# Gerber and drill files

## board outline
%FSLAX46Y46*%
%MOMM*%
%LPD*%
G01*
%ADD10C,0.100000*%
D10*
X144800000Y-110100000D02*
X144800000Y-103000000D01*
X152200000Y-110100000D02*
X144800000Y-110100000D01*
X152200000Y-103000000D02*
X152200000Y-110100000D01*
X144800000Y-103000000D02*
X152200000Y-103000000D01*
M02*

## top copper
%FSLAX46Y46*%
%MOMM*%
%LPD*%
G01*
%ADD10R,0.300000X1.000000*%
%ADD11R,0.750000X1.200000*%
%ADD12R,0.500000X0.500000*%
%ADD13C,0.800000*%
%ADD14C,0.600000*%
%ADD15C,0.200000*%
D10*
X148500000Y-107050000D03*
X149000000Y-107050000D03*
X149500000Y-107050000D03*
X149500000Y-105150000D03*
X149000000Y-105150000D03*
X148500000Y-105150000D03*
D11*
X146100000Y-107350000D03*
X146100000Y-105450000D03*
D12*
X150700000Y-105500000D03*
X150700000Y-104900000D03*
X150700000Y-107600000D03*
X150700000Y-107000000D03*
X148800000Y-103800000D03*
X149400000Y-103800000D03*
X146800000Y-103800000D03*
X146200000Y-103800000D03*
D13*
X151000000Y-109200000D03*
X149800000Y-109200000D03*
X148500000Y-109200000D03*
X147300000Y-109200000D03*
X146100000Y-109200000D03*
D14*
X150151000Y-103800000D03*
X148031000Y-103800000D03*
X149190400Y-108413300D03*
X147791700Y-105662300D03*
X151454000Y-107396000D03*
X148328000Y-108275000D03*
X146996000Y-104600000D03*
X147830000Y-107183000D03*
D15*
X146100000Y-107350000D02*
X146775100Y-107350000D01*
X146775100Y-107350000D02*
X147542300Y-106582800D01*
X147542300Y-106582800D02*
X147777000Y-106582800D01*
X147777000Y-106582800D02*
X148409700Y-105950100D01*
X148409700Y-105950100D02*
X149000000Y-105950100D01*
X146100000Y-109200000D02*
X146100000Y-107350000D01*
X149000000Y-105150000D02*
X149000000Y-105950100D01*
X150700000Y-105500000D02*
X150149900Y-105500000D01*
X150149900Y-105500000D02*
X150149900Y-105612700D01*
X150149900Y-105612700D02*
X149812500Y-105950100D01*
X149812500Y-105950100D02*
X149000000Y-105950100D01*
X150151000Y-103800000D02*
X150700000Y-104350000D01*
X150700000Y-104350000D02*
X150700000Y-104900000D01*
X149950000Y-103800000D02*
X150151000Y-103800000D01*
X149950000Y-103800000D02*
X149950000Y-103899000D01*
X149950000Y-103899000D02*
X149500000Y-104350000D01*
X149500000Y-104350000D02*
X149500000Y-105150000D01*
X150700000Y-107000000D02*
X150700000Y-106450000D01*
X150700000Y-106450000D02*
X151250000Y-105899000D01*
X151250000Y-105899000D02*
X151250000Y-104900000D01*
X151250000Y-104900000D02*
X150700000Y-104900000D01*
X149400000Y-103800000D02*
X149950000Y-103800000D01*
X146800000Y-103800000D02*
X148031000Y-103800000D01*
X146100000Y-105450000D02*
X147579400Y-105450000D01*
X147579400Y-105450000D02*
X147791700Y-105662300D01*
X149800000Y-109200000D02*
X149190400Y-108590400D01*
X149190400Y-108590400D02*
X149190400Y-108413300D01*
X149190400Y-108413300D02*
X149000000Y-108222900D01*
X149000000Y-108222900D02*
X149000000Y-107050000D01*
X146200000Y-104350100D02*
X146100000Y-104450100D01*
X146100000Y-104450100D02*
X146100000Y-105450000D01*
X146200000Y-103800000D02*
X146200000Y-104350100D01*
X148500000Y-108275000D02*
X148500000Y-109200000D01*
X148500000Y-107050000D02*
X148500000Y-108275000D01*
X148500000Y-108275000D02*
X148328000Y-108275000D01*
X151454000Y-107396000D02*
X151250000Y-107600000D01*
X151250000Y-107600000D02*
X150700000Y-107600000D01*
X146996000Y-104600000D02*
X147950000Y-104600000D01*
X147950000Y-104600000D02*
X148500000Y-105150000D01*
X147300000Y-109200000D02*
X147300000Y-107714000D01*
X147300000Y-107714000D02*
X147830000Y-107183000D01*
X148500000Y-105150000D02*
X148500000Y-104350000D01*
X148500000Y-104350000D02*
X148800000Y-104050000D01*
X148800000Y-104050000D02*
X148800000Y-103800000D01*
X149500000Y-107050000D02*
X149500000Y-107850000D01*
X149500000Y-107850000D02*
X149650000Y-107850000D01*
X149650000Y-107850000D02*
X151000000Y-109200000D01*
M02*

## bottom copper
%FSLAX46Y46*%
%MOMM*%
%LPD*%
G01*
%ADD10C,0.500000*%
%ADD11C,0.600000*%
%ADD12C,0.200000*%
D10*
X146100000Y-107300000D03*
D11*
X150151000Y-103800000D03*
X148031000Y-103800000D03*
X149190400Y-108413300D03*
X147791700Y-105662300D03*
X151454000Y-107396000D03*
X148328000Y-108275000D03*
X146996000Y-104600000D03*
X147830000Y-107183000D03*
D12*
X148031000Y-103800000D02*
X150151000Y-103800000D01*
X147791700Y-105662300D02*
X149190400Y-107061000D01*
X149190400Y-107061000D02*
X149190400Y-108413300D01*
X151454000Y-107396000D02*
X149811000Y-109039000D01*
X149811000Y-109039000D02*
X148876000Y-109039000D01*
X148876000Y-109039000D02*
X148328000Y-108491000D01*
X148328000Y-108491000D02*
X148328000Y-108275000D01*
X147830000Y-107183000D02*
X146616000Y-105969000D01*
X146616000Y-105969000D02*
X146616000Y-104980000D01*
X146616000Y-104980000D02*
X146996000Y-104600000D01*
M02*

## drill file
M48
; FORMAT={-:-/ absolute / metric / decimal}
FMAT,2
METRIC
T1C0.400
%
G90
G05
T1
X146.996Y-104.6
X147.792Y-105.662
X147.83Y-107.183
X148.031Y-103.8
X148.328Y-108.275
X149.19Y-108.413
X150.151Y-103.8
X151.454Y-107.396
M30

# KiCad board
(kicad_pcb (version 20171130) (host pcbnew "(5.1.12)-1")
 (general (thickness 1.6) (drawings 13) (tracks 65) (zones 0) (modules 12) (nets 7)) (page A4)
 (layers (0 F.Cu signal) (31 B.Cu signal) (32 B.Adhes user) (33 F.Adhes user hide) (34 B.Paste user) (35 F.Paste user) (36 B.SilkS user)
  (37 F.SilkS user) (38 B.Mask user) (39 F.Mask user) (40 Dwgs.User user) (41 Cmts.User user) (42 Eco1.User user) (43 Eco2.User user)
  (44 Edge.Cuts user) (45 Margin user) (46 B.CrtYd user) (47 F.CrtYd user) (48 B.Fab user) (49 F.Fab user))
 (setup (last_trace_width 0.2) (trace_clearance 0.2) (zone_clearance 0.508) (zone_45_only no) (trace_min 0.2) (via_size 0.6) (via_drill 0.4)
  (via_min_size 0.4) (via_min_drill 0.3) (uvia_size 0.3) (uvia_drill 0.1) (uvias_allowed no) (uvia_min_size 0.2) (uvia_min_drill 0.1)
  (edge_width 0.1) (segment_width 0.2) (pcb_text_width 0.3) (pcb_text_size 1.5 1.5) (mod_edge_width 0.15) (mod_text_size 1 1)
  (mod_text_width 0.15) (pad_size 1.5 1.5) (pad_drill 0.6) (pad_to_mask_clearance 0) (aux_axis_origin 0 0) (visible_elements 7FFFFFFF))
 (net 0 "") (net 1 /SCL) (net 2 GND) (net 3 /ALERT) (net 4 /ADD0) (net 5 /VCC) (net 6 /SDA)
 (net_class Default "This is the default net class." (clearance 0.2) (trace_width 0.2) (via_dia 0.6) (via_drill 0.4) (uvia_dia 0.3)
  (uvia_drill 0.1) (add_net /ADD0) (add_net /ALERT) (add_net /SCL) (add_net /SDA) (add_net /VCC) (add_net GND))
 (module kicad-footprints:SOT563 (layer F.Cu) (at 149 106.1)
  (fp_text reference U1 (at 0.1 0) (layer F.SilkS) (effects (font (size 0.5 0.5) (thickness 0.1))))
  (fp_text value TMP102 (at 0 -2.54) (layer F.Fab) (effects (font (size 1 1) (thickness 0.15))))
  (pad 1 smd rect (at -0.5 0.95) (size 0.3 1) (layers F.Cu F.Paste F.Mask) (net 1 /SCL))
  (pad 2 smd rect (at 0 0.95) (size 0.3 1) (layers F.Cu F.Paste F.Mask) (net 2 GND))
  (pad 3 smd rect (at 0.5 0.95) (size 0.3 1) (layers F.Cu F.Paste F.Mask) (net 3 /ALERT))
  (pad 4 smd rect (at 0.5 -0.95) (size 0.3 1) (layers F.Cu F.Paste F.Mask) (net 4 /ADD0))
  (pad 5 smd rect (at 0 -0.95) (size 0.3 1) (layers F.Cu F.Paste F.Mask) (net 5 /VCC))
  (pad 6 smd rect (at -0.5 -0.95) (size 0.3 1) (layers F.Cu F.Paste F.Mask) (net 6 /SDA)))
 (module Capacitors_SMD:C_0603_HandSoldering (layer F.Cu) (at 146.1 106.4 90)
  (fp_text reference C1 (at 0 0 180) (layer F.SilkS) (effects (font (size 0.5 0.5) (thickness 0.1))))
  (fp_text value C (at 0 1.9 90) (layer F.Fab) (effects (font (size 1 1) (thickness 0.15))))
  (pad 1 smd rect (at -0.95 0 90) (size 1.2 0.75) (layers F.Cu F.Paste F.Mask) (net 5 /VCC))
  (pad 2 smd rect (at 0.95 0 90) (size 1.2 0.75) (layers F.Cu F.Paste F.Mask) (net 2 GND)))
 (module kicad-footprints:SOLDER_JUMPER (layer F.Cu) (at 150.7 105.2 90)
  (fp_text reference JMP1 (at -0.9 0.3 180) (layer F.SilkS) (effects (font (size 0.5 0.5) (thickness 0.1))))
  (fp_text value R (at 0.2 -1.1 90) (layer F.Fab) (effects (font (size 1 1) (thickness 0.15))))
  (pad 1 smd rect (at -0.3 0 90) (size 0.5 0.5) (layers F.Cu F.Paste F.Mask) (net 5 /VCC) (clearance 0.05))
  (pad 2 smd rect (at 0.3 0 90) (size 0.5 0.5) (layers F.Cu F.Paste F.Mask) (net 4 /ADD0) (clearance 0.05)))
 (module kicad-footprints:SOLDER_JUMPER (layer F.Cu) (at 150.7 107.3 90)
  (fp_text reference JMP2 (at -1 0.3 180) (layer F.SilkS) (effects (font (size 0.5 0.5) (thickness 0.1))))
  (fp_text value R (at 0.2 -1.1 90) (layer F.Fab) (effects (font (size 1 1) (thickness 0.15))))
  (pad 1 smd rect (at -0.3 0 90) (size 0.5 0.5) (layers F.Cu F.Paste F.Mask) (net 1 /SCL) (clearance 0.05))
  (pad 2 smd rect (at 0.3 0 90) (size 0.5 0.5) (layers F.Cu F.Paste F.Mask) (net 4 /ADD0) (clearance 0.05)))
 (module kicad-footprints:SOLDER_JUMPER (layer F.Cu) (at 149.1 103.8)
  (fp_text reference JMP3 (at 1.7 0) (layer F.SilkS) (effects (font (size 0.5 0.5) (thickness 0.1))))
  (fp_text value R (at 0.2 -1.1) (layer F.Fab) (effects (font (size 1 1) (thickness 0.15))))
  (pad 1 smd rect (at -0.3 0) (size 0.5 0.5) (layers F.Cu F.Paste F.Mask) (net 6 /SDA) (clearance 0.05))
  (pad 2 smd rect (at 0.3 0) (size 0.5 0.5) (layers F.Cu F.Paste F.Mask) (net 4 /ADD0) (clearance 0.05)))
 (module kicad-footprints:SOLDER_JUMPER (layer F.Cu) (at 146.5 103.8 180)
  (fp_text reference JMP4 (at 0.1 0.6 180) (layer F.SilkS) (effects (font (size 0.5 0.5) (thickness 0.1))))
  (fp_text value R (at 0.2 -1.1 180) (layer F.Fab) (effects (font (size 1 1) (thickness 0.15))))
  (pad 1 smd rect (at -0.3 0 180) (size 0.5 0.5) (layers F.Cu F.Paste F.Mask) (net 4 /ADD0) (clearance 0.05))
  (pad 2 smd rect (at 0.3 0 180) (size 0.5 0.5) (layers F.Cu F.Paste F.Mask) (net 2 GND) (clearance 0.05)))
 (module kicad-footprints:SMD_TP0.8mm (layer F.Cu) (at 151 109.2)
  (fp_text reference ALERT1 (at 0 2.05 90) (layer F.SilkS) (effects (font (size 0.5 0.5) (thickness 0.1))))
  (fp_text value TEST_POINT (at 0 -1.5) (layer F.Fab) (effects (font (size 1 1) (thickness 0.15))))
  (pad 1 smd circle (at 0 0) (size 0.8 0.8) (layers F.Cu F.Paste F.Mask) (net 3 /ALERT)))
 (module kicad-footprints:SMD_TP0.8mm (layer F.Cu) (at 149.8 109.2)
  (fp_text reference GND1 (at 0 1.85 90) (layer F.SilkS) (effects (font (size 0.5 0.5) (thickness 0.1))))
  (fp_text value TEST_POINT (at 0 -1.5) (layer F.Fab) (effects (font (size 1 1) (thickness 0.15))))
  (pad 1 smd circle (at 0 0) (size 0.8 0.8) (layers F.Cu F.Paste F.Mask) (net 2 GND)))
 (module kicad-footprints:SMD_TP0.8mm (layer F.Cu) (at 148.5 109.2)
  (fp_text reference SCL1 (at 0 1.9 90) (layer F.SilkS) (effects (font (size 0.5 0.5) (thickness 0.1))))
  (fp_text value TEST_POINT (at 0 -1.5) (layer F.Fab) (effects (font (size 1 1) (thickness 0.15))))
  (pad 1 smd circle (at 0 0) (size 0.8 0.8) (layers F.Cu F.Paste F.Mask) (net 1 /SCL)))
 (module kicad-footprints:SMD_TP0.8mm (layer F.Cu) (at 147.3 109.2)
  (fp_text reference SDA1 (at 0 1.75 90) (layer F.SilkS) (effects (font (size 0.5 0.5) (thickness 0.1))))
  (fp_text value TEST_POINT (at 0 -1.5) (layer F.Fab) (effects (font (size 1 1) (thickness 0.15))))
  (pad 1 smd circle (at 0 0) (size 0.8 0.8) (layers F.Cu F.Paste F.Mask) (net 6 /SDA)))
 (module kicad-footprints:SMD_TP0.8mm (layer F.Cu) (at 146.1 109.2)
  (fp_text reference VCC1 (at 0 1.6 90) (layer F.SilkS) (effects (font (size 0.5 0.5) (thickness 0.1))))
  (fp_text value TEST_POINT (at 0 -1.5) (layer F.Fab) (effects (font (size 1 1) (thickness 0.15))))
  (pad 1 smd circle (at 0 0) (size 0.8 0.8) (layers F.Cu F.Paste F.Mask) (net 5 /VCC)))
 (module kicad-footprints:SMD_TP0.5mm (layer B.Cu) (at 146.1 107.3)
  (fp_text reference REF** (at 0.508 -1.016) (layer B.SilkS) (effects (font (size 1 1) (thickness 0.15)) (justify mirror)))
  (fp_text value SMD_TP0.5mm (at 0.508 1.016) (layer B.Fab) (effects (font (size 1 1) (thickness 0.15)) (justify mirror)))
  (pad 1 smd circle (at 0 0) (size 0.5 0.5) (layers B.Cu B.Paste B.Mask)))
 (gr_line (start 144.8 110.1) (end 144.8 103) (angle 90) (layer Edge.Cuts) (width 0.1))
 (gr_line (start 152.2 110.1) (end 144.8 110.1) (angle 90) (layer Edge.Cuts) (width 0.1))
 (gr_line (start 152.2 103) (end 152.2 110.1) (angle 90) (layer Edge.Cuts) (width 0.1))
 (gr_line (start 144.8 103) (end 152.2 103) (angle 90) (layer Edge.Cuts) (width 0.1))
 (segment (start 146.1 107.35) (end 146.7751 107.35) (width 0.2) (layer F.Cu) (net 5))
 (segment (start 146.7751 107.35) (end 147.5423 106.5828) (width 0.2) (layer F.Cu) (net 5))
 (segment (start 147.5423 106.5828) (end 147.777 106.5828) (width 0.2) (layer F.Cu) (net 5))
 (segment (start 147.777 106.5828) (end 148.4097 105.9501) (width 0.2) (layer F.Cu) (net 5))
 (segment (start 148.4097 105.9501) (end 149 105.9501) (width 0.2) (layer F.Cu) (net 5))
 (segment (start 146.1 109.2) (end 146.1 107.35) (width 0.2) (layer F.Cu) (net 5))
 (segment (start 149 105.15) (end 149 105.9501) (width 0.2) (layer F.Cu) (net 5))
 (segment (start 150.7 105.5) (end 150.1499 105.5) (width 0.2) (layer F.Cu) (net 5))
 (segment (start 150.1499 105.5) (end 150.1499 105.6127) (width 0.2) (layer F.Cu) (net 5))
 (segment (start 150.1499 105.6127) (end 149.8125 105.9501) (width 0.2) (layer F.Cu) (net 5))
 (segment (start 149.8125 105.9501) (end 149 105.9501) (width 0.2) (layer F.Cu) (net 5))
 (segment (start 150.151 103.8) (end 150.7 104.35) (width 0.2) (layer F.Cu) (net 4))
 (segment (start 150.7 104.35) (end 150.7 104.9) (width 0.2) (layer F.Cu) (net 4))
 (segment (start 149.95 103.8) (end 150.151 103.8) (width 0.2) (layer F.Cu) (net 4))
 (segment (start 149.95 103.8) (end 149.95 103.899) (width 0.2) (layer F.Cu) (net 4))
 (segment (start 149.95 103.899) (end 149.5 104.35) (width 0.2) (layer F.Cu) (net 4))
 (segment (start 149.5 104.35) (end 149.5 105.15) (width 0.2) (layer F.Cu) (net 4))
 (segment (start 150.7 107) (end 150.7 106.45) (width 0.2) (layer F.Cu) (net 4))
 (segment (start 150.7 106.45) (end 151.25 105.899) (width 0.2) (layer F.Cu) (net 4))
 (segment (start 151.25 105.899) (end 151.25 104.9) (width 0.2) (layer F.Cu) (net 4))
 (segment (start 151.25 104.9) (end 150.7 104.9) (width 0.2) (layer F.Cu) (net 4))
 (segment (start 149.4 103.8) (end 149.95 103.8) (width 0.2) (layer F.Cu) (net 4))
 (segment (start 146.8 103.8) (end 148.031 103.8) (width 0.2) (layer F.Cu) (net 4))
 (segment (start 148.031 103.8) (end 150.151 103.8) (width 0.2) (layer B.Cu) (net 4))
 (via (at 150.151 103.8) (size 0.6) (layers F.Cu B.Cu) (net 4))
 (via (at 148.031 103.8) (size 0.6) (layers F.Cu B.Cu) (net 4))
 (segment (start 146.1 105.45) (end 147.5794 105.45) (width 0.2) (layer F.Cu) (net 2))
 (segment (start 147.5794 105.45) (end 147.7917 105.6623) (width 0.2) (layer F.Cu) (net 2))
 (segment (start 149.8 109.2) (end 149.1904 108.5904) (width 0.2) (layer F.Cu) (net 2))
 (segment (start 149.1904 108.5904) (end 149.1904 108.4133) (width 0.2) (layer F.Cu) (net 2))
 (segment (start 149.1904 108.4133) (end 149 108.2229) (width 0.2) (layer F.Cu) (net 2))
 (segment (start 149 108.2229) (end 149 107.05) (width 0.2) (layer F.Cu) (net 2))
 (segment (start 147.7917 105.6623) (end 149.1904 107.061) (width 0.2) (layer B.Cu) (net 2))
 (segment (start 149.1904 107.061) (end 149.1904 108.4133) (width 0.2) (layer B.Cu) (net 2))
 (segment (start 146.2 104.3501) (end 146.1 104.4501) (width 0.2) (layer F.Cu) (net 2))
 (segment (start 146.1 104.4501) (end 146.1 105.45) (width 0.2) (layer F.Cu) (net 2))
 (segment (start 146.2 103.8) (end 146.2 104.3501) (width 0.2) (layer F.Cu) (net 2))
 (via (at 149.1904 108.4133) (size 0.6) (layers F.Cu B.Cu) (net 2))
 (via (at 147.7917 105.6623) (size 0.6) (layers F.Cu B.Cu) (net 2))
 (segment (start 148.5 108.275) (end 148.5 109.2) (width 0.2) (layer F.Cu) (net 1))
 (segment (start 148.5 107.05) (end 148.5 108.275) (width 0.2) (layer F.Cu) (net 1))
 (segment (start 148.5 108.275) (end 148.328 108.275) (width 0.2) (layer F.Cu) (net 1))
 (segment (start 151.454 107.396) (end 149.811 109.039) (width 0.2) (layer B.Cu) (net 1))
 (segment (start 149.811 109.039) (end 148.876 109.039) (width 0.2) (layer B.Cu) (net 1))
 (segment (start 148.876 109.039) (end 148.328 108.491) (width 0.2) (layer B.Cu) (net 1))
 (segment (start 148.328 108.491) (end 148.328 108.275) (width 0.2) (layer B.Cu) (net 1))
 (segment (start 151.454 107.396) (end 151.25 107.6) (width 0.2) (layer F.Cu) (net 1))
 (segment (start 151.25 107.6) (end 150.7 107.6) (width 0.2) (layer F.Cu) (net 1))
 (via (at 151.454 107.396) (size 0.6) (layers F.Cu B.Cu) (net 1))
 (via (at 148.328 108.275) (size 0.6) (layers F.Cu B.Cu) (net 1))
 (segment (start 146.996 104.6) (end 147.95 104.6) (width 0.2) (layer F.Cu) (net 6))
 (segment (start 147.95 104.6) (end 148.5 105.15) (width 0.2) (layer F.Cu) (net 6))
 (segment (start 147.83 107.183) (end 146.616 105.969) (width 0.2) (layer B.Cu) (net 6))
 (segment (start 146.616 105.969) (end 146.616 104.98) (width 0.2) (layer B.Cu) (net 6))
 (segment (start 146.616 104.98) (end 146.996 104.6) (width 0.2) (layer B.Cu) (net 6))
 (segment (start 147.3 109.2) (end 147.3 107.714) (width 0.2) (layer F.Cu) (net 6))
 (segment (start 147.3 107.714) (end 147.83 107.183) (width 0.2) (layer F.Cu) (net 6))
 (segment (start 148.5 105.15) (end 148.5 104.35) (width 0.2) (layer F.Cu) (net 6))
 (segment (start 148.5 104.35) (end 148.8 104.05) (width 0.2) (layer F.Cu) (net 6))
 (segment (start 148.8 104.05) (end 148.8 103.8) (width 0.2) (layer F.Cu) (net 6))
 (via (at 146.996 104.6) (size 0.6) (layers F.Cu B.Cu) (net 6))
 (via (at 147.83 107.183) (size 0.6) (layers F.Cu B.Cu) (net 6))
 (segment (start 149.5 107.05) (end 149.5 107.85) (width 0.2) (layer F.Cu) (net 3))
 (segment (start 149.5 107.85) (end 149.65 107.85) (width 0.2) (layer F.Cu) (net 3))
 (segment (start 149.65 107.85) (end 151 109.2) (width 0.2) (layer F.Cu) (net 3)))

